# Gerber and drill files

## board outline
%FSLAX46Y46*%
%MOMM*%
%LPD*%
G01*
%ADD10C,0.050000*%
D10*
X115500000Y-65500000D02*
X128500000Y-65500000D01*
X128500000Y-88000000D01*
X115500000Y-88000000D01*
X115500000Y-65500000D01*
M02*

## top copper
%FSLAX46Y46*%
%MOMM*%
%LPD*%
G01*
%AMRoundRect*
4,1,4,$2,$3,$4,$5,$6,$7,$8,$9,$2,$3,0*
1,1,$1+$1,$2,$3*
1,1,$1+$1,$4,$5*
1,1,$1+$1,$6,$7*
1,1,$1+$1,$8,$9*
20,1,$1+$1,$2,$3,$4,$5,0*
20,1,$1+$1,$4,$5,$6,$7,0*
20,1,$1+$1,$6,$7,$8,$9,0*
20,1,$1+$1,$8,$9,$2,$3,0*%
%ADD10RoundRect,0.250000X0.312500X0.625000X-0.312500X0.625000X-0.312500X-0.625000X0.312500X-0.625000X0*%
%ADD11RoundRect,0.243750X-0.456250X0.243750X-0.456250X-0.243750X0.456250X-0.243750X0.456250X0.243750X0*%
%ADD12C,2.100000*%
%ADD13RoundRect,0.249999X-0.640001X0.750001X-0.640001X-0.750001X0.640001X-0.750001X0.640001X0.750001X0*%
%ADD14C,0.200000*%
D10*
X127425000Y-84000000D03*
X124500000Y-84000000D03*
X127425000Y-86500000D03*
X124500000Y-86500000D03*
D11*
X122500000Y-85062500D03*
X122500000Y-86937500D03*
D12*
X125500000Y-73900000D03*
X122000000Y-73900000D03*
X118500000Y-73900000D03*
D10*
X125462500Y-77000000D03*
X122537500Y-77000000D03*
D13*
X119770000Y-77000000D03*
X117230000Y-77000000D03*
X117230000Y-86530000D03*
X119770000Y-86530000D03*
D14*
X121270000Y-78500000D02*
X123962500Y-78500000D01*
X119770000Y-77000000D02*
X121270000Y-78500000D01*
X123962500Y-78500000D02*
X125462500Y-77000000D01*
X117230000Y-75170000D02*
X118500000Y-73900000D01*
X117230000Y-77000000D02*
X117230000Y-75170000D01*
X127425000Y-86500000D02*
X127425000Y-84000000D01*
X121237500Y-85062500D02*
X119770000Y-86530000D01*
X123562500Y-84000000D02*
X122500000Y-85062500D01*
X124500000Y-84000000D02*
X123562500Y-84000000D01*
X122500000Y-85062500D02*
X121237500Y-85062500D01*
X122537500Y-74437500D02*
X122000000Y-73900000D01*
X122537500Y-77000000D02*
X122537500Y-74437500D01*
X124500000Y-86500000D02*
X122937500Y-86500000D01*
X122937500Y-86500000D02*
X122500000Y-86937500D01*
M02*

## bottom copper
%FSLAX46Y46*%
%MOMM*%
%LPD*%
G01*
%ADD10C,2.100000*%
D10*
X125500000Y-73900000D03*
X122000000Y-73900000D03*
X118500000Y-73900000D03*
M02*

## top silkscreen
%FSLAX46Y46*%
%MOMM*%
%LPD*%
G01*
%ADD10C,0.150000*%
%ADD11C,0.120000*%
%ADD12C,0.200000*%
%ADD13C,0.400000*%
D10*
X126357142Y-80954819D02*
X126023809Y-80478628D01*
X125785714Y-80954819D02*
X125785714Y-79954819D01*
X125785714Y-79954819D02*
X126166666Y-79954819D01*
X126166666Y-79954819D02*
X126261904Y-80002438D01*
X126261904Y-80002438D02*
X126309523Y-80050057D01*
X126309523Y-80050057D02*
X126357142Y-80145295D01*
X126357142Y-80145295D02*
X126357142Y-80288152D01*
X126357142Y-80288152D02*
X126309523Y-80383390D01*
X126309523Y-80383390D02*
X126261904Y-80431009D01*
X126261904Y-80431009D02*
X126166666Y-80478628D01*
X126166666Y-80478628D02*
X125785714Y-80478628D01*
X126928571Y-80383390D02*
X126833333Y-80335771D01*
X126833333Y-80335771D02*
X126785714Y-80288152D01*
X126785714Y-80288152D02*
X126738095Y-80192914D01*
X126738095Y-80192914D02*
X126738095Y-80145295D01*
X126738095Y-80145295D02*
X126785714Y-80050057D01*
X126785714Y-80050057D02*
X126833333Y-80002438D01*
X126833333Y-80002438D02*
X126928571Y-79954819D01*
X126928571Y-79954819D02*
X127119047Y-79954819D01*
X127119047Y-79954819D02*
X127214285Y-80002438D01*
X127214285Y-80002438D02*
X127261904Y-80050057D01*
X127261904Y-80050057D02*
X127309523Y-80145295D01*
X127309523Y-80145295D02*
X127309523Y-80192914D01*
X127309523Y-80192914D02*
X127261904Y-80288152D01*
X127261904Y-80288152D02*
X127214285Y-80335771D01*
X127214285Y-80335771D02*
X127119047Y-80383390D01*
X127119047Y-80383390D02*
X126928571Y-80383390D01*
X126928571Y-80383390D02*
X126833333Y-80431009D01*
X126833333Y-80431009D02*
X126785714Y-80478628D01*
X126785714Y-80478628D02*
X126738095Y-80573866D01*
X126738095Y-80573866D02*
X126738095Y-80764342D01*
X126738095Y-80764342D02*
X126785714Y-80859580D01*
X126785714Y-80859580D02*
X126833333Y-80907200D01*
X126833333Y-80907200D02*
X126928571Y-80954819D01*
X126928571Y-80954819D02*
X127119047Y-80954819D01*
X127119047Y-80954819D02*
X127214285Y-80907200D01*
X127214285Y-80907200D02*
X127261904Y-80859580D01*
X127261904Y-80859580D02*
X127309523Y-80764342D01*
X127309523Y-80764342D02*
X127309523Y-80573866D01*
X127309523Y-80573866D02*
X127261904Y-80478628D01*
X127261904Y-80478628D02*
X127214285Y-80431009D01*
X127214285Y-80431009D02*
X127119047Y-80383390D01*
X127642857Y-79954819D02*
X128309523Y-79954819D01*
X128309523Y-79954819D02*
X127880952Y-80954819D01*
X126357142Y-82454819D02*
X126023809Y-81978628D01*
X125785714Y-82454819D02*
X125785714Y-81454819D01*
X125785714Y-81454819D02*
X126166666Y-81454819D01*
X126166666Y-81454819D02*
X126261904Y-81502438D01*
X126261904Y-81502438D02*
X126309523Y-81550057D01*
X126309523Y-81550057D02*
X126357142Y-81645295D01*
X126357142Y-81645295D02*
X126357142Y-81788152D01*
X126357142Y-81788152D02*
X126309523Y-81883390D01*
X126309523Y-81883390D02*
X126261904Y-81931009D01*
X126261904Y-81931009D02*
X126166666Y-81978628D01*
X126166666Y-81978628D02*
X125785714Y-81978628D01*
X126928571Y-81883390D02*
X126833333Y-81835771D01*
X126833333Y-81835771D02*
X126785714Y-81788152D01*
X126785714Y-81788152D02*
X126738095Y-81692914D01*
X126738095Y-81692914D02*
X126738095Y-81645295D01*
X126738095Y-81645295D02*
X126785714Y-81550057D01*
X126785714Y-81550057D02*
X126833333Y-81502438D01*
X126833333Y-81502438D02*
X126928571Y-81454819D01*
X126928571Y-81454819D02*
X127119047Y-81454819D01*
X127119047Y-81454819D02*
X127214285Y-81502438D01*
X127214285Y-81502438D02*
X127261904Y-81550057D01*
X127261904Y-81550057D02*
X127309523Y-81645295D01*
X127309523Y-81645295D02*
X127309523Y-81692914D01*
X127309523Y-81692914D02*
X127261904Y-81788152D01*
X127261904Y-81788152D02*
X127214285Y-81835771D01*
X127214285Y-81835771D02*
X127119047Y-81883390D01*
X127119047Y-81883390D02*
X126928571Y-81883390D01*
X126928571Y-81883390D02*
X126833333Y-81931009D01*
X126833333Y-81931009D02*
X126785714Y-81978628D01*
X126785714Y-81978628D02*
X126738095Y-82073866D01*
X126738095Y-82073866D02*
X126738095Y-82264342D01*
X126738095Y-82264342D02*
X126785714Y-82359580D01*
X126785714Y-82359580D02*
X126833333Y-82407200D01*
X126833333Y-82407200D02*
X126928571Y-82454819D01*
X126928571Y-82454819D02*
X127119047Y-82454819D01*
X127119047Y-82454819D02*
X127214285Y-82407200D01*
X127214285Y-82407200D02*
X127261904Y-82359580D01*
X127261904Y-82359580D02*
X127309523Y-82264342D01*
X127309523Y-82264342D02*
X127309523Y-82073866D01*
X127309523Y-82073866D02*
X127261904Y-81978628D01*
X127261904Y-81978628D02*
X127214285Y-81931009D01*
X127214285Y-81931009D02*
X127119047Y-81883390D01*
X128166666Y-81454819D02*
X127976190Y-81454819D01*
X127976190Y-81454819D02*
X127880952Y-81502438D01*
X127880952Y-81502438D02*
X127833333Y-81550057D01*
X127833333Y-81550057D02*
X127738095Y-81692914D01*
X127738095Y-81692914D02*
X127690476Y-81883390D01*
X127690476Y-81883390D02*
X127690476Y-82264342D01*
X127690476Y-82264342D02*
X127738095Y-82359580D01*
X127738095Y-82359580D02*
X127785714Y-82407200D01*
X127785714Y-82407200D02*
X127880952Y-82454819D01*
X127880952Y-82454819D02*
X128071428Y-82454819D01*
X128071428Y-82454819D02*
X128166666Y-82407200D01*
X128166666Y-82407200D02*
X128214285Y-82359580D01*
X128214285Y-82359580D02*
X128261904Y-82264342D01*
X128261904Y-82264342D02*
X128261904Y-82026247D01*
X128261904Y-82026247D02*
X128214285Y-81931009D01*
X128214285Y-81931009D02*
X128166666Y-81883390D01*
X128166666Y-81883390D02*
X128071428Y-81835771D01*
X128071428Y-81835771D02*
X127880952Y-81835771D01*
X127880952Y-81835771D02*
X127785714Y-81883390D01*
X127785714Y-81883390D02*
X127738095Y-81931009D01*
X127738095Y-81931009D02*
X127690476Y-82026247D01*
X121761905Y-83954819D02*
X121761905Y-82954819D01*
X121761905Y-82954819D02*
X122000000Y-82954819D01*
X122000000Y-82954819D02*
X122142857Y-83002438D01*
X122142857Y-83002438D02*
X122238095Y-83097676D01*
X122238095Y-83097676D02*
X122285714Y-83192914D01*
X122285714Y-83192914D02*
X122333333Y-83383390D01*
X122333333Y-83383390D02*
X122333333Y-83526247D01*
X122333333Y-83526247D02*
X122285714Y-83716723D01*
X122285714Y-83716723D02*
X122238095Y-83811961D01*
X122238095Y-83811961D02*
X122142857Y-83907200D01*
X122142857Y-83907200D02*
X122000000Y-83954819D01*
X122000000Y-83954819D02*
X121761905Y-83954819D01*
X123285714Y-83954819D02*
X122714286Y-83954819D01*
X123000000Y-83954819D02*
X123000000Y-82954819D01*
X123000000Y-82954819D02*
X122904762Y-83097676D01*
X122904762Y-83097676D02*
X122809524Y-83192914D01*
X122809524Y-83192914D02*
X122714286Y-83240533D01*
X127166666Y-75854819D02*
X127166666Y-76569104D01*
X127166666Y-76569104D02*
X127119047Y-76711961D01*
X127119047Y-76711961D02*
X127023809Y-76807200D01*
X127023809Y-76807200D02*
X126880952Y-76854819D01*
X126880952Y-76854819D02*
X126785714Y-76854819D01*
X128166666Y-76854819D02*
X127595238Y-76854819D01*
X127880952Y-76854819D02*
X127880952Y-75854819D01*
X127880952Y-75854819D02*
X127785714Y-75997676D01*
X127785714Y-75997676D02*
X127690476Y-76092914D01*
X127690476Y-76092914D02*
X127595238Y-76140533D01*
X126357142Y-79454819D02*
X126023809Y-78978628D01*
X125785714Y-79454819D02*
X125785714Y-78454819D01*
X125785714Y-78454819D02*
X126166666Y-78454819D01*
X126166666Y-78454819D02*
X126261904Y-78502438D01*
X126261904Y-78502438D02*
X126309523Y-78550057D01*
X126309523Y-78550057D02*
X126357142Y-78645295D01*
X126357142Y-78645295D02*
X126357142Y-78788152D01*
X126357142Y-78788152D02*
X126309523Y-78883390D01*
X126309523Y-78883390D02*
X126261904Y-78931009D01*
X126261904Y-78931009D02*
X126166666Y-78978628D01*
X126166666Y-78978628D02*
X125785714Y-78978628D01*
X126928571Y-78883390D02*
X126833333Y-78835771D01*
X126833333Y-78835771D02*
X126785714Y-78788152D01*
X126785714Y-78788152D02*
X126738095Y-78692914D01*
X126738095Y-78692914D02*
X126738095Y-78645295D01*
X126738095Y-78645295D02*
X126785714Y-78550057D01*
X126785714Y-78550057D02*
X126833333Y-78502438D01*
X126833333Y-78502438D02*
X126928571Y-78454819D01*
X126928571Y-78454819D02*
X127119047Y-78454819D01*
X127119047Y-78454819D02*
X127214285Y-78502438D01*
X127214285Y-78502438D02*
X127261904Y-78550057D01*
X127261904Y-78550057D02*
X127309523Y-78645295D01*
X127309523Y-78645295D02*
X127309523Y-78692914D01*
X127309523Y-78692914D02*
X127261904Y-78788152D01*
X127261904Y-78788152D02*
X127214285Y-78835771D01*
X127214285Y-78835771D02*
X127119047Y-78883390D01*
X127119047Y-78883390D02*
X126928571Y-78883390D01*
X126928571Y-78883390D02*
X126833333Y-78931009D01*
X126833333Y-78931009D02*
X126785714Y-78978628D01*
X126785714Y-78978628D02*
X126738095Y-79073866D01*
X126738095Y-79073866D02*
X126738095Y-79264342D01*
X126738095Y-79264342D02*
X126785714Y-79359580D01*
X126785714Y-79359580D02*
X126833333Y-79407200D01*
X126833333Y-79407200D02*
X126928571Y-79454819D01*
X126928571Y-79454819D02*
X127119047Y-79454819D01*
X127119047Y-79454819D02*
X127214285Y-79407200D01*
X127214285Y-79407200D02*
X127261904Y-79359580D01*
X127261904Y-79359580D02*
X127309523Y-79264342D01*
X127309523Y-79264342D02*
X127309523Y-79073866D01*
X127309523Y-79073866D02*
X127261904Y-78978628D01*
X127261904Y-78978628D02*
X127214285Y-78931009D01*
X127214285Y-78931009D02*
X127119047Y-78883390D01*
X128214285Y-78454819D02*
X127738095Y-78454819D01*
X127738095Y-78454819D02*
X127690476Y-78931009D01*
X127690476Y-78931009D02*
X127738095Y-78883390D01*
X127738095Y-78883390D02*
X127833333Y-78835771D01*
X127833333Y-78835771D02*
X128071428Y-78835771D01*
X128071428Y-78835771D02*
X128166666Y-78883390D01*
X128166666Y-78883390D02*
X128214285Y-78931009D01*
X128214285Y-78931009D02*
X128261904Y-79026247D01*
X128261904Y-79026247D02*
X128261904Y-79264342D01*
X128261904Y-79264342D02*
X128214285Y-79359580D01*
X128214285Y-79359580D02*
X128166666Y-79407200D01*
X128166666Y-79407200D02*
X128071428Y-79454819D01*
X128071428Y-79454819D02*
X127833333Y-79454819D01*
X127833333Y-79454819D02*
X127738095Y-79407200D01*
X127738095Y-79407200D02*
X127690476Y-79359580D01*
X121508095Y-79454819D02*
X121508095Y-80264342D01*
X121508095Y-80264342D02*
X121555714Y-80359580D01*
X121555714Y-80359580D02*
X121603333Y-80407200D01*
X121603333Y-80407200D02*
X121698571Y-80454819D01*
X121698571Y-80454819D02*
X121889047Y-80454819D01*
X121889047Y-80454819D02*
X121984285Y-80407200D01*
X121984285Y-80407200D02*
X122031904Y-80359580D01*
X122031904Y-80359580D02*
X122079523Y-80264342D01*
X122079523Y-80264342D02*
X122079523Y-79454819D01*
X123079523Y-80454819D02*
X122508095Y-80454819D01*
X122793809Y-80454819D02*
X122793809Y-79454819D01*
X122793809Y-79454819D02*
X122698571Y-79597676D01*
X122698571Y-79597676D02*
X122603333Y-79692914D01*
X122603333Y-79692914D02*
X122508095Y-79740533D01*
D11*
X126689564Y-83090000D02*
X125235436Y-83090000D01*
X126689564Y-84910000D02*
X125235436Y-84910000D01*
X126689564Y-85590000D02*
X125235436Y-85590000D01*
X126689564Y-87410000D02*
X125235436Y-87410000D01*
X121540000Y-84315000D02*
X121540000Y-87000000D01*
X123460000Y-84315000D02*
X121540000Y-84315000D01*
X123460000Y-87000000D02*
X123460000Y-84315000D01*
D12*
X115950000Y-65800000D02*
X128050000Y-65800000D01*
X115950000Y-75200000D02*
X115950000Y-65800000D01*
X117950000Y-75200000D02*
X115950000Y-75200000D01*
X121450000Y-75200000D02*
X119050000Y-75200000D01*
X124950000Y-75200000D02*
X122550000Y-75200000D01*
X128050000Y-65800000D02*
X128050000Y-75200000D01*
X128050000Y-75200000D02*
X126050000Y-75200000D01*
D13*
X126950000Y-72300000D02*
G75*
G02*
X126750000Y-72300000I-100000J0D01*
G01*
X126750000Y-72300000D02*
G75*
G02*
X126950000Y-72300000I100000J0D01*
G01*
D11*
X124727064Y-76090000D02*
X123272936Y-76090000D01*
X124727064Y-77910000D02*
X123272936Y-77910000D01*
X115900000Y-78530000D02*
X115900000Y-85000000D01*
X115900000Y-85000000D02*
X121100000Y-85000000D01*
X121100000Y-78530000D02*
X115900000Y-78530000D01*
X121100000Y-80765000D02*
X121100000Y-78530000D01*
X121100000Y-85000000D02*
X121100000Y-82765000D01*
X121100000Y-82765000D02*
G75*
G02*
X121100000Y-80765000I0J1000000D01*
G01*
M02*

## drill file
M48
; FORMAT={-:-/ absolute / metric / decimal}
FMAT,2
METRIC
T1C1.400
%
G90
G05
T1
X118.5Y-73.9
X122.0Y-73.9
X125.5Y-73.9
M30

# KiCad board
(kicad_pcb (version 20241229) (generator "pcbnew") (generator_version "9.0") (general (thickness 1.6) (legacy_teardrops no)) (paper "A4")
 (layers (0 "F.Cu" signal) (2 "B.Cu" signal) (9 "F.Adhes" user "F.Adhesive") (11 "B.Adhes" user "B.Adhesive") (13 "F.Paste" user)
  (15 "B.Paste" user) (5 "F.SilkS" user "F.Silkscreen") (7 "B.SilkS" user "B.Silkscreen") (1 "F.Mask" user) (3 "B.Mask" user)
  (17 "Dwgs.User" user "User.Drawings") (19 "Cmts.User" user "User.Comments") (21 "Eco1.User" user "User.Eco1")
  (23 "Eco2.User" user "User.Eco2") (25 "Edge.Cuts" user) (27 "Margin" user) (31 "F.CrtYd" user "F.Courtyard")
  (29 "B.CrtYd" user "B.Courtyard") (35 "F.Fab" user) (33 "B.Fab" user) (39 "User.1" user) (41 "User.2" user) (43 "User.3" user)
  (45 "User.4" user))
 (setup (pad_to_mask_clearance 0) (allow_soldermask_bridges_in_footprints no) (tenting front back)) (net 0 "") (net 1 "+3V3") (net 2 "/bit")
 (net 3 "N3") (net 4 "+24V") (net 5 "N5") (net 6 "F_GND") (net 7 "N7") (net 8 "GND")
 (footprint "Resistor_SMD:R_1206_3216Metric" (layer "F.Cu") (at 125.9625 84 180)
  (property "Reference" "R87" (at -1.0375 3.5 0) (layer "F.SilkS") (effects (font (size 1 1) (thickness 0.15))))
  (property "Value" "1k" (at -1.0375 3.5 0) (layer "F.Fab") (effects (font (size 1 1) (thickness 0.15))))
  (fp_line (start -0.727064 0.91) (end 0.727064 0.91) (stroke (width 0.12) (type solid)) (layer "F.SilkS"))
  (fp_line (start -0.727064 -0.91) (end 0.727064 -0.91) (stroke (width 0.12) (type solid)) (layer "F.SilkS"))
  (pad "1" smd roundrect (at -1.4625 0 180) (size 1.125 1.75) (layers "F.Cu" "F.Mask" "F.Paste") (roundrect_rratio 0.222222) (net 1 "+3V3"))
  (pad "2" smd roundrect (at 1.4625 0 180) (size 1.125 1.75) (layers "F.Cu" "F.Mask" "F.Paste") (roundrect_rratio 0.222222) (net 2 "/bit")))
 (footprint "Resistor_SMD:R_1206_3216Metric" (layer "F.Cu") (at 125.9625 86.5 180)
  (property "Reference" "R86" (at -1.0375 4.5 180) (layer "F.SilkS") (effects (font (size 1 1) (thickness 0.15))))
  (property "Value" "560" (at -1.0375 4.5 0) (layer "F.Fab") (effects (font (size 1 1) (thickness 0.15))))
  (fp_line (start -0.727064 0.91) (end 0.727064 0.91) (stroke (width 0.12) (type solid)) (layer "F.SilkS"))
  (fp_line (start -0.727064 -0.91) (end 0.727064 -0.91) (stroke (width 0.12) (type solid)) (layer "F.SilkS"))
  (pad "1" smd roundrect (at -1.4625 0 180) (size 1.125 1.75) (layers "F.Cu" "F.Mask" "F.Paste") (roundrect_rratio 0.222222) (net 1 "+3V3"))
  (pad "2" smd roundrect (at 1.4625 0 180) (size 1.125 1.75) (layers "F.Cu" "F.Mask" "F.Paste") (roundrect_rratio 0.222222) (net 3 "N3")))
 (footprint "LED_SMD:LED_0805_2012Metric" (layer "F.Cu") (at 122.5 86 -90)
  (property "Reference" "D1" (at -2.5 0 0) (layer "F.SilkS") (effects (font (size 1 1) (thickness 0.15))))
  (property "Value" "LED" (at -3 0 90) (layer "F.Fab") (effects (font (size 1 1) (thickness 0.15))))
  (fp_line (start -1.685 0.96) (end 1 0.96) (stroke (width 0.12) (type solid)) (layer "F.SilkS"))
  (fp_line (start -1.685 -0.96) (end -1.685 0.96) (stroke (width 0.12) (type solid)) (layer "F.SilkS"))
  (fp_line (start 1 -0.96) (end -1.685 -0.96) (stroke (width 0.12) (type solid)) (layer "F.SilkS"))
  (pad "1" smd roundrect (at -0.9375 0 270) (size 0.975 1.4) (layers "F.Cu" "F.Mask" "F.Paste") (roundrect_rratio 0.25) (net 2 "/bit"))
  (pad "2" smd roundrect (at 0.9375 0 270) (size 0.975 1.4) (layers "F.Cu" "F.Mask" "F.Paste") (roundrect_rratio 0.25) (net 3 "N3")))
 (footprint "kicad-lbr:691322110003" (layer "F.Cu") (at 122 73.9 180)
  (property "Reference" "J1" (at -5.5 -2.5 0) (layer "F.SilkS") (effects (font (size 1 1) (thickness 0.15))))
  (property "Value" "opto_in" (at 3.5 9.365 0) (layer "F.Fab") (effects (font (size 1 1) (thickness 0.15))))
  (fp_line (start 6.05 8.1) (end -6.05 8.1) (stroke (width 0.2) (type solid)) (layer "F.SilkS"))
  (fp_line (start 6.05 -1.3) (end 6.05 8.1) (stroke (width 0.2) (type solid)) (layer "F.SilkS"))
  (fp_line (start 4.05 -1.3) (end 6.05 -1.3) (stroke (width 0.2) (type solid)) (layer "F.SilkS"))
  (fp_line (start 0.55 -1.3) (end 2.95 -1.3) (stroke (width 0.2) (type solid)) (layer "F.SilkS"))
  (fp_line (start -2.95 -1.3) (end -0.55 -1.3) (stroke (width 0.2) (type solid)) (layer "F.SilkS"))
  (fp_line (start -6.05 8.1) (end -6.05 -1.3) (stroke (width 0.2) (type solid)) (layer "F.SilkS"))
  (fp_line (start -6.05 -1.3) (end -4.05 -1.3) (stroke (width 0.2) (type solid)) (layer "F.SilkS"))
  (fp_circle (center -4.85 1.6) (end -4.75 1.6) (stroke (width 0.4) (type solid)) (fill no) (layer "F.SilkS"))
  (pad "1" thru_hole circle (at -3.5 0 180) (size 2.1 2.1) (drill 1.4) (layers "*.Cu" "*.Mask") (remove_unused_layers no) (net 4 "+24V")
   (solder_mask_margin 0.102))
  (pad "2" thru_hole circle (at 0 0 180) (size 2.1 2.1) (drill 1.4) (layers "*.Cu" "*.Mask") (remove_unused_layers no) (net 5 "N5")
   (solder_mask_margin 0.102))
  (pad "3" thru_hole circle (at 3.5 0 180) (size 2.1 2.1) (drill 1.4) (layers "*.Cu" "*.Mask") (remove_unused_layers no) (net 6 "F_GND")
   (solder_mask_margin 0.102)))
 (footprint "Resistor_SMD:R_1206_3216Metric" (layer "F.Cu") (at 124 77 180)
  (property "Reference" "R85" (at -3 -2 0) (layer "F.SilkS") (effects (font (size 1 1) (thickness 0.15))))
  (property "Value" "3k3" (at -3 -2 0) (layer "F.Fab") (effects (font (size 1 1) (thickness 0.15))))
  (fp_line (start -0.727064 0.91) (end 0.727064 0.91) (stroke (width 0.12) (type solid)) (layer "F.SilkS"))
  (fp_line (start -0.727064 -0.91) (end 0.727064 -0.91) (stroke (width 0.12) (type solid)) (layer "F.SilkS"))
  (pad "1" smd roundrect (at -1.4625 0 180) (size 1.125 1.75) (layers "F.Cu" "F.Mask" "F.Paste") (roundrect_rratio 0.222222) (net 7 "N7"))
  (pad "2" smd roundrect (at 1.4625 0 180) (size 1.125 1.75) (layers "F.Cu" "F.Mask" "F.Paste") (roundrect_rratio 0.222222) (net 5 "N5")))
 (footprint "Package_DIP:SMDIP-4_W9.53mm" (layer "F.Cu") (at 118.5 81.765 -90)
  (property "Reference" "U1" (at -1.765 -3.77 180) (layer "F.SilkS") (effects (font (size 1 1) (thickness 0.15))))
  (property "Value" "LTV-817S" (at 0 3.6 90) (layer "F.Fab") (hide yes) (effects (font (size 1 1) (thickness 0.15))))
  (fp_line (start -3.235 2.6) (end 3.235 2.6) (stroke (width 0.12) (type solid)) (layer "F.SilkS"))
  (fp_line (start 3.235 2.6) (end 3.235 -2.6) (stroke (width 0.12) (type solid)) (layer "F.SilkS"))
  (fp_line (start -3.235 -2.6) (end -3.235 2.6) (stroke (width 0.12) (type solid)) (layer "F.SilkS"))
  (fp_line (start -1 -2.6) (end -3.235 -2.6) (stroke (width 0.12) (type solid)) (layer "F.SilkS"))
  (fp_line (start 3.235 -2.6) (end 1 -2.6) (stroke (width 0.12) (type solid)) (layer "F.SilkS"))
  (fp_arc (start 1 -2.6) (mid 0 -1.6) (end -1 -2.6) (stroke (width 0.12) (type solid)) (layer "F.SilkS"))
  (pad "1" smd roundrect (at -4.765 -1.27 270) (size 2 1.78) (layers "F.Cu" "F.Mask" "F.Paste") (roundrect_rratio 0.140449) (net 7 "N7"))
  (pad "2" smd roundrect (at -4.765 1.27 270) (size 2 1.78) (layers "F.Cu" "F.Mask" "F.Paste") (roundrect_rratio 0.140449) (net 6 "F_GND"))
  (pad "3" smd roundrect (at 4.765 1.27 270) (size 2 1.78) (layers "F.Cu" "F.Mask" "F.Paste") (roundrect_rratio 0.140449) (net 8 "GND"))
  (pad "4" smd roundrect (at 4.765 -1.27 270) (size 2 1.78) (layers "F.Cu" "F.Mask" "F.Paste") (roundrect_rratio 0.140449) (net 2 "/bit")))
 (gr_rect (start 115.5 65.5) (end 128.5 88) (stroke (width 0.05) (type default)) (fill no) (layer "Edge.Cuts"))
 (segment (start 121.27 78.5) (end 123.9625 78.5) (width 0.2) (layer "F.Cu") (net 7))
 (segment (start 119.77 77) (end 121.27 78.5) (width 0.2) (layer "F.Cu") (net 7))
 (segment (start 123.9625 78.5) (end 125.4625 77) (width 0.2) (layer "F.Cu") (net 7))
 (segment (start 117.23 75.17) (end 118.5 73.9) (width 0.2) (layer "F.Cu") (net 6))
 (segment (start 117.23 77) (end 117.23 75.17) (width 0.2) (layer "F.Cu") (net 6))
 (segment (start 127.425 86.5) (end 127.425 84) (width 0.2) (layer "F.Cu") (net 1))
 (segment (start 121.2375 85.0625) (end 119.77 86.53) (width 0.2) (layer "F.Cu") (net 2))
 (segment (start 123.5625 84) (end 122.5 85.0625) (width 0.2) (layer "F.Cu") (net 2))
 (segment (start 124.5 84) (end 123.5625 84) (width 0.2) (layer "F.Cu") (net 2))
 (segment (start 122.5 85.0625) (end 121.2375 85.0625) (width 0.2) (layer "F.Cu") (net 2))
 (segment (start 122.5375 74.4375) (end 122 73.9) (width 0.2) (layer "F.Cu") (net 5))
 (segment (start 122.5375 77) (end 122.5375 74.4375) (width 0.2) (layer "F.Cu") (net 5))
 (segment (start 124.5 86.5) (end 122.9375 86.5) (width 0.2) (layer "F.Cu") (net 3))
 (segment (start 122.9375 86.5) (end 122.5 86.9375) (width 0.2) (layer "F.Cu") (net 3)))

